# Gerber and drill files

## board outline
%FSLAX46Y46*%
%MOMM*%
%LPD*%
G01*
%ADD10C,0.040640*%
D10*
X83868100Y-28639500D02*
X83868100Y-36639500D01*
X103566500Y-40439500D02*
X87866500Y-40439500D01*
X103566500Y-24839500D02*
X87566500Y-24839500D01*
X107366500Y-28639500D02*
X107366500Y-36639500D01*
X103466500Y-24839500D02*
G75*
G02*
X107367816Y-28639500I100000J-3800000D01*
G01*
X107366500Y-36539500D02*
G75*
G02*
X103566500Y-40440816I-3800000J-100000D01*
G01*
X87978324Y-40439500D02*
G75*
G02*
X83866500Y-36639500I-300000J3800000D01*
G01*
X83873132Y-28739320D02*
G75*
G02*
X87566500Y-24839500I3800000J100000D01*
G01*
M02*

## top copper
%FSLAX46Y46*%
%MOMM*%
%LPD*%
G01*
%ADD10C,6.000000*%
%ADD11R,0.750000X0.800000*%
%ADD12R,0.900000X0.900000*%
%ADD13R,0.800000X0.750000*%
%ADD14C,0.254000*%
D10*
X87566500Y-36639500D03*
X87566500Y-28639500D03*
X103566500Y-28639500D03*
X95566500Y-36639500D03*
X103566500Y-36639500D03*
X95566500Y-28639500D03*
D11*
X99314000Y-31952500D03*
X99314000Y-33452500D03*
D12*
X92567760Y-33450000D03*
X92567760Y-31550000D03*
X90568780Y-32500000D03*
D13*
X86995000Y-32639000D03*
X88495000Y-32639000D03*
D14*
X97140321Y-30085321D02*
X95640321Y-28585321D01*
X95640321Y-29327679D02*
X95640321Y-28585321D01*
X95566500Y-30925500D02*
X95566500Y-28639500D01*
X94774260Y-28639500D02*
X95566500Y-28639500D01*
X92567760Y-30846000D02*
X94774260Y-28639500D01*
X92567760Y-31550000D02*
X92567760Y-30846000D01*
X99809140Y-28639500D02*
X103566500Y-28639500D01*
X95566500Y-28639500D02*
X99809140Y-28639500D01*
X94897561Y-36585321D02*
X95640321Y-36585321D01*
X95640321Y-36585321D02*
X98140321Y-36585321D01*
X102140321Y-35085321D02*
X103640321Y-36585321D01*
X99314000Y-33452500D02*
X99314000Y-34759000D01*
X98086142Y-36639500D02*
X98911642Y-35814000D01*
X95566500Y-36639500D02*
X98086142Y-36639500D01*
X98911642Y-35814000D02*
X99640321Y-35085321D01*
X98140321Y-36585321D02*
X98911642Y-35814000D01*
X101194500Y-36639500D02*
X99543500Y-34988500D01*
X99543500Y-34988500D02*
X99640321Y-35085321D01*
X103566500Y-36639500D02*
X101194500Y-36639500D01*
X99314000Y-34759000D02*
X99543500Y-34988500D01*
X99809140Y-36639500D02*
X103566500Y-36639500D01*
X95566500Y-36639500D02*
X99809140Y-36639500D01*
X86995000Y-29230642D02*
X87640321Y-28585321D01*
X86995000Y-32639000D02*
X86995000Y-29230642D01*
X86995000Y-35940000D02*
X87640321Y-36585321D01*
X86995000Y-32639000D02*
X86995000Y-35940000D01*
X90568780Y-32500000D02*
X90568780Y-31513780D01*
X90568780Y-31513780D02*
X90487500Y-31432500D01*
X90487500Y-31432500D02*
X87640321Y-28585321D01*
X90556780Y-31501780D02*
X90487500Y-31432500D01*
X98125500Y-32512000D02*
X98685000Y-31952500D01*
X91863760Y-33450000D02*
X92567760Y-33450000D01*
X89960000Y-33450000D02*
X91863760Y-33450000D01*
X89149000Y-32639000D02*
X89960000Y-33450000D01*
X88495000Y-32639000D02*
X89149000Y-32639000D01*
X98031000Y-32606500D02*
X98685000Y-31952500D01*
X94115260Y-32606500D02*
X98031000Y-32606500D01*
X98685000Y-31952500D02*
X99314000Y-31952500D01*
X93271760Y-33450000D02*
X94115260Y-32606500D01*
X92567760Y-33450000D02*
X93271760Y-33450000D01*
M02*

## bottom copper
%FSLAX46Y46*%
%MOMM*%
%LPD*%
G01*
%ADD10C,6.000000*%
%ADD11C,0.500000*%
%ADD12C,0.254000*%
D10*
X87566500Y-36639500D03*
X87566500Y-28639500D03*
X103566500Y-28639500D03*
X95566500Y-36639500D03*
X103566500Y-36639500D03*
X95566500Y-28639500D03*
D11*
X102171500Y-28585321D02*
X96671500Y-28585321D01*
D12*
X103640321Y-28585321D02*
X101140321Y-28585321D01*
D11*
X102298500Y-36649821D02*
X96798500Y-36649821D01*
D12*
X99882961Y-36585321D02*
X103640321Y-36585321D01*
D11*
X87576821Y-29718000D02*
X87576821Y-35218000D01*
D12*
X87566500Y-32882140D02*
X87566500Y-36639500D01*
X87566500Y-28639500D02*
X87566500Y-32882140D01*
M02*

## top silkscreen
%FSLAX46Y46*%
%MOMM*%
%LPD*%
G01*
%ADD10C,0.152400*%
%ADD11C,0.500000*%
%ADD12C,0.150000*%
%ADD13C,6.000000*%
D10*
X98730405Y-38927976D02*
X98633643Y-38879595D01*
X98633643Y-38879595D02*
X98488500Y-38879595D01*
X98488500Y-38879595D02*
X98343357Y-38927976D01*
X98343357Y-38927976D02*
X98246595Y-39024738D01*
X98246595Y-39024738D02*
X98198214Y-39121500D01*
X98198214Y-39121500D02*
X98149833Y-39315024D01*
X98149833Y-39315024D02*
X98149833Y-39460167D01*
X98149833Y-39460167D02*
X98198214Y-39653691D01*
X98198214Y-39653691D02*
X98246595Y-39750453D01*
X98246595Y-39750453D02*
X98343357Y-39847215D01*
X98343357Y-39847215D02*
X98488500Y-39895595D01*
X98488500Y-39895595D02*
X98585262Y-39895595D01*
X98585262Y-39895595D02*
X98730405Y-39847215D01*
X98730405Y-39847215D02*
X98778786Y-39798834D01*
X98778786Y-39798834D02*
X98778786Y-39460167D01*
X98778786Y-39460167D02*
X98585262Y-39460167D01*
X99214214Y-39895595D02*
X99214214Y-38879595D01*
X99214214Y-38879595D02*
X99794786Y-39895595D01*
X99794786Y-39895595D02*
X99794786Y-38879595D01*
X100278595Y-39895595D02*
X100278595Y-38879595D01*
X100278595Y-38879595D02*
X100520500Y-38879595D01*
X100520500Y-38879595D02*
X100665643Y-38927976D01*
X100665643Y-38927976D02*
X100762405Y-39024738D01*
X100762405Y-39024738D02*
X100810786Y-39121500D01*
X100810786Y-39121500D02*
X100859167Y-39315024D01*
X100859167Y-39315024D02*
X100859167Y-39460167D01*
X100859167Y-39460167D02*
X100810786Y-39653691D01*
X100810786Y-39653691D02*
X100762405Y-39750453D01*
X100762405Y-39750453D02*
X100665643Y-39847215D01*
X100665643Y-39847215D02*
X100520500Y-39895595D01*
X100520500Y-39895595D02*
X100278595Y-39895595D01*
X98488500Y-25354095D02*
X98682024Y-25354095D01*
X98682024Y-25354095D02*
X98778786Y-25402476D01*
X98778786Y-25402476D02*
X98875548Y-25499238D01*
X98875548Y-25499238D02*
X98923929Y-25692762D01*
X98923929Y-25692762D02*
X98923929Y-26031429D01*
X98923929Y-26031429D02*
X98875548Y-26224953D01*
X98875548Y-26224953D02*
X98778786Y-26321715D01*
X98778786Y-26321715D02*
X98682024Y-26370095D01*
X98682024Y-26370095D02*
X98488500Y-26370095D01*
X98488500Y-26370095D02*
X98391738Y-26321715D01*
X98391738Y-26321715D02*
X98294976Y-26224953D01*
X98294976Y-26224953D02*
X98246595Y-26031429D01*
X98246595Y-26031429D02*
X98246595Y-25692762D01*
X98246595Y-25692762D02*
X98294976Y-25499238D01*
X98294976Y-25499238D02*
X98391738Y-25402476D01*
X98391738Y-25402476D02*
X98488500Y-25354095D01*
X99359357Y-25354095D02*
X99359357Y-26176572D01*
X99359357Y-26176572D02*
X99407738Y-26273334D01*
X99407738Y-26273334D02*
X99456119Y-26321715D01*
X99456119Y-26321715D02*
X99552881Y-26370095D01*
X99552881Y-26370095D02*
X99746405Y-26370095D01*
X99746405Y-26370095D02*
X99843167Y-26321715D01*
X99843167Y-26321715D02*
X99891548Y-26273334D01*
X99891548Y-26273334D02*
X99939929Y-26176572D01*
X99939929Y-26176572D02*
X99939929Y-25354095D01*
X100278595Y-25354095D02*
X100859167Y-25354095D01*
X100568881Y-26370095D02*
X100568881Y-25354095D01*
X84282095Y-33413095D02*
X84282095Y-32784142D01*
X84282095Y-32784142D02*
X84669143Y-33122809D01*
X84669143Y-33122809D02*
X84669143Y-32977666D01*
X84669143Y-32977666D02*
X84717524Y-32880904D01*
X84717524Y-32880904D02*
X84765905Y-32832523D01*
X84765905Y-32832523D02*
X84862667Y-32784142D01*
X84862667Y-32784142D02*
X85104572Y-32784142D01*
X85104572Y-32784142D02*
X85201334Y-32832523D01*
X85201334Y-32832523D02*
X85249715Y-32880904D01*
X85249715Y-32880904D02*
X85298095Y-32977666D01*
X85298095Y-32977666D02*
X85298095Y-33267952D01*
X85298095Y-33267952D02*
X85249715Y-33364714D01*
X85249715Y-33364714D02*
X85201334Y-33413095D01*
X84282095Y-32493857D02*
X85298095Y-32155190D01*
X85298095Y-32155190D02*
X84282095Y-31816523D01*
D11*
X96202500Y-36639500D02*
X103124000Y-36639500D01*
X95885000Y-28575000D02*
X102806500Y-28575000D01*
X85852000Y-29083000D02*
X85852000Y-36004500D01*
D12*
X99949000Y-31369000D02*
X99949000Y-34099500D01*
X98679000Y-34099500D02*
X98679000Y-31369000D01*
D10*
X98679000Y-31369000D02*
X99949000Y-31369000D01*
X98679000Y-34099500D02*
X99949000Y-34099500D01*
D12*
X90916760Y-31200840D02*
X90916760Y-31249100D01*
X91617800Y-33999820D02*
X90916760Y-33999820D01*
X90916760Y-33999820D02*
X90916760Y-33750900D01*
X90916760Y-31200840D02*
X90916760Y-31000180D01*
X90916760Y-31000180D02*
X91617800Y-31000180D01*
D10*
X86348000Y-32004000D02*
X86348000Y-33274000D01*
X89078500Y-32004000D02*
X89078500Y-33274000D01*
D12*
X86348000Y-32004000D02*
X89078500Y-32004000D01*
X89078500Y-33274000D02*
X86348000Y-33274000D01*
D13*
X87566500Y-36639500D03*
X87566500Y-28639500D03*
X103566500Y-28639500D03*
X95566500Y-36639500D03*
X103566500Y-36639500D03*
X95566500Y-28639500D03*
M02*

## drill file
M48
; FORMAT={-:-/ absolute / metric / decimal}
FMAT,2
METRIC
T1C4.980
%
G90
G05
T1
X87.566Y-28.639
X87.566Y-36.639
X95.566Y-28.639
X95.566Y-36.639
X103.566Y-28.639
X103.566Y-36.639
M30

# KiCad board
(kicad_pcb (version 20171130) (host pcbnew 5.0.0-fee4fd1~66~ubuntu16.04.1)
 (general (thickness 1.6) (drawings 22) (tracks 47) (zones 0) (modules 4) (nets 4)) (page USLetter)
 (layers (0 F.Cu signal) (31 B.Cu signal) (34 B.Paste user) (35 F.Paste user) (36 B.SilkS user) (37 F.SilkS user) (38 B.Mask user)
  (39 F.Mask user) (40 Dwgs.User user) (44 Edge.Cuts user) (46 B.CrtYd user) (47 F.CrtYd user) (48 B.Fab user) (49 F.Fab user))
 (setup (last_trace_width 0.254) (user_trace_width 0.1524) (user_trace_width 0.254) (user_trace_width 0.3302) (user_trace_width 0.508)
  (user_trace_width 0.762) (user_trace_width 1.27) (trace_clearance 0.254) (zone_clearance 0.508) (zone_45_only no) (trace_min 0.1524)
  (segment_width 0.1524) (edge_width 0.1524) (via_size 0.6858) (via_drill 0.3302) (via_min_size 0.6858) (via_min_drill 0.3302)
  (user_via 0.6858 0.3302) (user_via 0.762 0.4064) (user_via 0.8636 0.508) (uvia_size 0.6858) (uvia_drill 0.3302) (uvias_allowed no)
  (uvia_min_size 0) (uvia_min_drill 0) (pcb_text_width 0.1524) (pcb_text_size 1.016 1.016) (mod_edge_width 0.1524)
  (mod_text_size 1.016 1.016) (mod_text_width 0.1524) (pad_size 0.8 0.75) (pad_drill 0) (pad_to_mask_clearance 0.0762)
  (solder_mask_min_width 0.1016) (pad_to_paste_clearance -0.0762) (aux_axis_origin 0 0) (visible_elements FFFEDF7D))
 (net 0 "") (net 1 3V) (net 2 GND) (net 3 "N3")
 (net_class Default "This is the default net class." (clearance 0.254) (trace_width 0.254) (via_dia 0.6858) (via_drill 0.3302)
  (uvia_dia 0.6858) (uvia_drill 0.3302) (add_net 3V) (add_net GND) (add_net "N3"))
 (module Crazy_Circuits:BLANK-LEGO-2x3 (layer F.Cu) (at 87.5665 36.6395)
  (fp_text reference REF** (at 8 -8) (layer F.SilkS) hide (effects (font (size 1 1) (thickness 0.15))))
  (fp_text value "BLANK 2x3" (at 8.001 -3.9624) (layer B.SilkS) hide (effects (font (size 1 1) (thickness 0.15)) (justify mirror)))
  (fp_line (start -3.6984 -8) (end -3.6984 0) (layer Edge.Cuts) (width 0.04064))
  (fp_line (start 16 3.8) (end 0.3 3.8) (layer Edge.Cuts) (width 0.04064))
  (fp_line (start 16 -11.8) (end 0 -11.8) (layer Edge.Cuts) (width 0.04064))
  (fp_line (start 19.8 -8) (end 19.8 0) (layer Edge.Cuts) (width 0.04064))
  (fp_arc (start 16 -8) (end 15.9 -11.8) (angle 91.50743576) (layer Edge.Cuts) (width 0.04064))
  (fp_arc (start 16 0) (end 19.8 -0.1) (angle 91.50743576) (layer Edge.Cuts) (width 0.04064))
  (fp_arc (start 0.111824 0) (end 0.411824 3.8) (angle 94.51398846) (layer Edge.Cuts) (width 0.04064))
  (fp_arc (start 0.106632 -8.00018) (end -3.693368 -7.90018) (angle 89.9) (layer Edge.Cuts) (width 0.04064))
  (pad + thru_hole circle (at 0 0) (size 6 6) (drill 4.98) (layers *.Cu F.SilkS B.Mask) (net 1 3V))
  (pad + thru_hole circle (at 0 -8) (size 6 6) (drill 4.98) (layers *.Cu F.SilkS B.Mask) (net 1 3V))
  (pad OUT thru_hole circle (at 16 -8) (size 6 6) (drill 4.98) (layers *.Cu *.Mask F.SilkS))
  (pad - thru_hole circle (at 8 0) (size 6 6) (drill 4.98) (layers *.Cu F.SilkS B.Mask) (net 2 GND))
  (pad - thru_hole circle (at 16 0) (size 6 6) (drill 4.98) (layers *.Cu *.Mask F.SilkS) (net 2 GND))
  (pad OUT thru_hole circle (at 8 -8) (size 6 6) (drill 4.98) (layers *.Cu F.SilkS B.Mask)))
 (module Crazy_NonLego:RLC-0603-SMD (layer F.Cu) (at 99.314 32.7025 90)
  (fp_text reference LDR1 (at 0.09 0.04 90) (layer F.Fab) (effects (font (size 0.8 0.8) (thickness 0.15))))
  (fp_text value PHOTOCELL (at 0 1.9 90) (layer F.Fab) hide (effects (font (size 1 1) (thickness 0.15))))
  (fp_line (start 1.3335 0.635) (end -1.397 0.635) (layer F.SilkS) (width 0.15))
  (fp_line (start -1.397 -0.635) (end 1.3335 -0.635) (layer F.SilkS) (width 0.15))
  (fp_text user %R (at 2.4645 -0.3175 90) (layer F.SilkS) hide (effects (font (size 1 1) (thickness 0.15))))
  (fp_line (start 1.3335 -0.635) (end 1.3335 0.635) (layer F.SilkS) (width 0.1524))
  (fp_line (start -1.397 -0.635) (end -1.397 0.635) (layer F.SilkS) (width 0.1524))
  (pad 2 smd rect (at 0.75 0 90) (size 0.8 0.75) (layers F.Cu F.Paste F.Mask) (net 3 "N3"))
  (pad 1 smd rect (at -0.75 0 90) (size 0.8 0.75) (layers F.Cu F.Paste F.Mask) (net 2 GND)))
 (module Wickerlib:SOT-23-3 (layer F.Cu) (at 91.567 32.5 90)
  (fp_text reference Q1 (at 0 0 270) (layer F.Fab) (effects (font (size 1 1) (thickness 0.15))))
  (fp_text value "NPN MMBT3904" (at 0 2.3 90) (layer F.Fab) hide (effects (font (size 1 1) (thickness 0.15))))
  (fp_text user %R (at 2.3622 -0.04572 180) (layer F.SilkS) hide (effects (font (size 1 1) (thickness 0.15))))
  (fp_line (start 1.29916 -0.65024) (end 1.2509 -0.65024) (layer F.SilkS) (width 0.15))
  (fp_line (start -1.49982 0.0508) (end -1.49982 -0.65024) (layer F.SilkS) (width 0.15))
  (fp_line (start -1.49982 -0.65024) (end -1.2509 -0.65024) (layer F.SilkS) (width 0.15))
  (fp_line (start 1.29916 -0.65024) (end 1.49982 -0.65024) (layer F.SilkS) (width 0.15))
  (fp_line (start 1.49982 -0.65024) (end 1.49982 0.0508) (layer F.SilkS) (width 0.15))
  (pad 1 smd rect (at -0.95 1.00076 90) (size 0.9 0.9) (layers F.Cu F.Paste F.Mask) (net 3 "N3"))
  (pad 2 smd rect (at 0.95 1.00076 90) (size 0.9 0.9) (layers F.Cu F.Paste F.Mask))
  (pad 3 smd rect (at 0 -0.99822 90) (size 0.9 0.9) (layers F.Cu F.Paste F.Mask) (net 1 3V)))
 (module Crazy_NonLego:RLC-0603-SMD (layer F.Cu) (at 87.745 32.639)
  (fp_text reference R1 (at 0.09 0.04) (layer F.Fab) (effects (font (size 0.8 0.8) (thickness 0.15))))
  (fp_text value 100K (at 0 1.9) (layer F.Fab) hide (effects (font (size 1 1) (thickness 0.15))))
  (fp_line (start -1.397 -0.635) (end -1.397 0.635) (layer F.SilkS) (width 0.1524))
  (fp_line (start 1.3335 -0.635) (end 1.3335 0.635) (layer F.SilkS) (width 0.1524))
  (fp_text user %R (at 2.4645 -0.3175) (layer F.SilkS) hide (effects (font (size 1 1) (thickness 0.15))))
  (fp_line (start -1.397 -0.635) (end 1.3335 -0.635) (layer F.SilkS) (width 0.15))
  (fp_line (start 1.3335 0.635) (end -1.397 0.635) (layer F.SilkS) (width 0.15))
  (pad 1 smd rect (at -0.75 0) (size 0.8 0.75) (layers F.Cu F.Paste F.Mask) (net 1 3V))
  (pad 2 smd rect (at 0.75 0) (size 0.8 0.75) (layers F.Cu F.Paste F.Mask) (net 3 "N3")))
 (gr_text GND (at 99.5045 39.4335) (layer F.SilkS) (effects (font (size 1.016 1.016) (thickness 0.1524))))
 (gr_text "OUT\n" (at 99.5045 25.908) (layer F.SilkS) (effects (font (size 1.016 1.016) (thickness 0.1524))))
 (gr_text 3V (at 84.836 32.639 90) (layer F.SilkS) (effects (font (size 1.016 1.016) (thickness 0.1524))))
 (gr_line (start 96.2025 36.6395) (end 103.124 36.6395) (layer F.SilkS) (width 0.5))
 (gr_line (start 95.885 28.575) (end 102.8065 28.575) (layer F.SilkS) (width 0.5))
 (gr_line (start 85.852 29.083) (end 85.852 36.0045) (layer F.SilkS) (width 0.5))
 (segment (start 97.140321 30.085321) (end 95.640321 28.585321) (width 0.254) (layer F.Cu) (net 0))
 (segment (start 95.640321 29.327679) (end 95.640321 28.585321) (width 0.254) (layer F.Cu) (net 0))
 (segment (start 102.1715 28.585321) (end 96.6715 28.585321) (width 0.5) (layer B.Cu) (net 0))
 (segment (start 103.640321 28.585321) (end 101.140321 28.585321) (width 0.254) (layer B.Cu) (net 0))
 (segment (start 95.5665 30.9255) (end 95.5665 28.6395) (width 0.254) (layer F.Cu) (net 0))
 (segment (start 94.77426 28.6395) (end 95.5665 28.6395) (width 0.254) (layer F.Cu) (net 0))
 (segment (start 92.56776 30.846) (end 94.77426 28.6395) (width 0.254) (layer F.Cu) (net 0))
 (segment (start 92.56776 31.55) (end 92.56776 30.846) (width 0.254) (layer F.Cu) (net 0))
 (segment (start 99.80914 28.6395) (end 103.5665 28.6395) (width 0.254) (layer F.Cu) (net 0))
 (segment (start 95.5665 28.6395) (end 99.80914 28.6395) (width 0.254) (layer F.Cu) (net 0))
 (segment (start 102.2985 36.649821) (end 96.7985 36.649821) (width 0.5) (layer B.Cu) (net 2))
 (segment (start 94.897561 36.585321) (end 95.640321 36.585321) (width 0.254) (layer F.Cu) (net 2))
 (segment (start 95.640321 36.585321) (end 98.140321 36.585321) (width 0.254) (layer F.Cu) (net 2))
 (segment (start 102.140321 35.085321) (end 103.640321 36.585321) (width 0.254) (layer F.Cu) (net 2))
 (segment (start 99.314 33.4525) (end 99.314 34.759) (width 0.254) (layer F.Cu) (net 2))
 (segment (start 98.086142 36.6395) (end 98.911642 35.814) (width 0.254) (layer F.Cu) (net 2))
 (segment (start 95.5665 36.6395) (end 98.086142 36.6395) (width 0.254) (layer F.Cu) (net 2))
 (segment (start 98.911642 35.814) (end 99.640321 35.085321) (width 0.254) (layer F.Cu) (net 2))
 (segment (start 98.140321 36.585321) (end 98.911642 35.814) (width 0.254) (layer F.Cu) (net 2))
 (segment (start 101.1945 36.6395) (end 99.5435 34.9885) (width 0.254) (layer F.Cu) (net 2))
 (segment (start 99.5435 34.9885) (end 99.640321 35.085321) (width 0.254) (layer F.Cu) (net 2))
 (segment (start 103.5665 36.6395) (end 101.1945 36.6395) (width 0.254) (layer F.Cu) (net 2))
 (segment (start 99.314 34.759) (end 99.5435 34.9885) (width 0.254) (layer F.Cu) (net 2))
 (segment (start 99.80914 36.6395) (end 103.5665 36.6395) (width 0.254) (layer F.Cu) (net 2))
 (segment (start 95.5665 36.6395) (end 99.80914 36.6395) (width 0.254) (layer F.Cu) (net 2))
 (segment (start 99.882961 36.585321) (end 103.640321 36.585321) (width 0.254) (layer B.Cu) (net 2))
 (segment (start 87.576821 29.718) (end 87.576821 35.218) (width 0.5) (layer B.Cu) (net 1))
 (segment (start 86.995 29.230642) (end 87.640321 28.585321) (width 0.254) (layer F.Cu) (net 1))
 (segment (start 86.995 32.639) (end 86.995 29.230642) (width 0.254) (layer F.Cu) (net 1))
 (segment (start 86.995 35.94) (end 87.640321 36.585321) (width 0.254) (layer F.Cu) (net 1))
 (segment (start 86.995 32.639) (end 86.995 35.94) (width 0.254) (layer F.Cu) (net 1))
 (segment (start 90.56878 32.5) (end 90.56878 31.51378) (width 0.254) (layer F.Cu) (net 1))
 (segment (start 90.56878 31.51378) (end 90.4875 31.4325) (width 0.254) (layer F.Cu) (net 1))
 (segment (start 90.4875 31.4325) (end 87.640321 28.585321) (width 0.254) (layer F.Cu) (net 1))
 (segment (start 90.55678 31.50178) (end 90.4875 31.4325) (width 0.254) (layer F.Cu) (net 1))
 (segment (start 87.5665 32.88214) (end 87.5665 36.6395) (width 0.254) (layer B.Cu) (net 1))
 (segment (start 87.5665 28.6395) (end 87.5665 32.88214) (width 0.254) (layer B.Cu) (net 1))
 (segment (start 98.1255 32.512) (end 98.685 31.9525) (width 0.254) (layer F.Cu) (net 3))
 (segment (start 91.86376 33.45) (end 92.56776 33.45) (width 0.254) (layer F.Cu) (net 3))
 (segment (start 89.96 33.45) (end 91.86376 33.45) (width 0.254) (layer F.Cu) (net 3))
 (segment (start 89.149 32.639) (end 89.96 33.45) (width 0.254) (layer F.Cu) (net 3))
 (segment (start 88.495 32.639) (end 89.149 32.639) (width 0.254) (layer F.Cu) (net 3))
 (segment (start 98.031 32.6065) (end 98.685 31.9525) (width 0.254) (layer F.Cu) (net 3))
 (segment (start 94.11526 32.6065) (end 98.031 32.6065) (width 0.254) (layer F.Cu) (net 3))
 (segment (start 98.685 31.9525) (end 99.314 31.9525) (width 0.254) (layer F.Cu) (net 3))
 (segment (start 93.27176 33.45) (end 94.11526 32.6065) (width 0.254) (layer F.Cu) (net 3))
 (segment (start 92.56776 33.45) (end 93.27176 33.45) (width 0.254) (layer F.Cu) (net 3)))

